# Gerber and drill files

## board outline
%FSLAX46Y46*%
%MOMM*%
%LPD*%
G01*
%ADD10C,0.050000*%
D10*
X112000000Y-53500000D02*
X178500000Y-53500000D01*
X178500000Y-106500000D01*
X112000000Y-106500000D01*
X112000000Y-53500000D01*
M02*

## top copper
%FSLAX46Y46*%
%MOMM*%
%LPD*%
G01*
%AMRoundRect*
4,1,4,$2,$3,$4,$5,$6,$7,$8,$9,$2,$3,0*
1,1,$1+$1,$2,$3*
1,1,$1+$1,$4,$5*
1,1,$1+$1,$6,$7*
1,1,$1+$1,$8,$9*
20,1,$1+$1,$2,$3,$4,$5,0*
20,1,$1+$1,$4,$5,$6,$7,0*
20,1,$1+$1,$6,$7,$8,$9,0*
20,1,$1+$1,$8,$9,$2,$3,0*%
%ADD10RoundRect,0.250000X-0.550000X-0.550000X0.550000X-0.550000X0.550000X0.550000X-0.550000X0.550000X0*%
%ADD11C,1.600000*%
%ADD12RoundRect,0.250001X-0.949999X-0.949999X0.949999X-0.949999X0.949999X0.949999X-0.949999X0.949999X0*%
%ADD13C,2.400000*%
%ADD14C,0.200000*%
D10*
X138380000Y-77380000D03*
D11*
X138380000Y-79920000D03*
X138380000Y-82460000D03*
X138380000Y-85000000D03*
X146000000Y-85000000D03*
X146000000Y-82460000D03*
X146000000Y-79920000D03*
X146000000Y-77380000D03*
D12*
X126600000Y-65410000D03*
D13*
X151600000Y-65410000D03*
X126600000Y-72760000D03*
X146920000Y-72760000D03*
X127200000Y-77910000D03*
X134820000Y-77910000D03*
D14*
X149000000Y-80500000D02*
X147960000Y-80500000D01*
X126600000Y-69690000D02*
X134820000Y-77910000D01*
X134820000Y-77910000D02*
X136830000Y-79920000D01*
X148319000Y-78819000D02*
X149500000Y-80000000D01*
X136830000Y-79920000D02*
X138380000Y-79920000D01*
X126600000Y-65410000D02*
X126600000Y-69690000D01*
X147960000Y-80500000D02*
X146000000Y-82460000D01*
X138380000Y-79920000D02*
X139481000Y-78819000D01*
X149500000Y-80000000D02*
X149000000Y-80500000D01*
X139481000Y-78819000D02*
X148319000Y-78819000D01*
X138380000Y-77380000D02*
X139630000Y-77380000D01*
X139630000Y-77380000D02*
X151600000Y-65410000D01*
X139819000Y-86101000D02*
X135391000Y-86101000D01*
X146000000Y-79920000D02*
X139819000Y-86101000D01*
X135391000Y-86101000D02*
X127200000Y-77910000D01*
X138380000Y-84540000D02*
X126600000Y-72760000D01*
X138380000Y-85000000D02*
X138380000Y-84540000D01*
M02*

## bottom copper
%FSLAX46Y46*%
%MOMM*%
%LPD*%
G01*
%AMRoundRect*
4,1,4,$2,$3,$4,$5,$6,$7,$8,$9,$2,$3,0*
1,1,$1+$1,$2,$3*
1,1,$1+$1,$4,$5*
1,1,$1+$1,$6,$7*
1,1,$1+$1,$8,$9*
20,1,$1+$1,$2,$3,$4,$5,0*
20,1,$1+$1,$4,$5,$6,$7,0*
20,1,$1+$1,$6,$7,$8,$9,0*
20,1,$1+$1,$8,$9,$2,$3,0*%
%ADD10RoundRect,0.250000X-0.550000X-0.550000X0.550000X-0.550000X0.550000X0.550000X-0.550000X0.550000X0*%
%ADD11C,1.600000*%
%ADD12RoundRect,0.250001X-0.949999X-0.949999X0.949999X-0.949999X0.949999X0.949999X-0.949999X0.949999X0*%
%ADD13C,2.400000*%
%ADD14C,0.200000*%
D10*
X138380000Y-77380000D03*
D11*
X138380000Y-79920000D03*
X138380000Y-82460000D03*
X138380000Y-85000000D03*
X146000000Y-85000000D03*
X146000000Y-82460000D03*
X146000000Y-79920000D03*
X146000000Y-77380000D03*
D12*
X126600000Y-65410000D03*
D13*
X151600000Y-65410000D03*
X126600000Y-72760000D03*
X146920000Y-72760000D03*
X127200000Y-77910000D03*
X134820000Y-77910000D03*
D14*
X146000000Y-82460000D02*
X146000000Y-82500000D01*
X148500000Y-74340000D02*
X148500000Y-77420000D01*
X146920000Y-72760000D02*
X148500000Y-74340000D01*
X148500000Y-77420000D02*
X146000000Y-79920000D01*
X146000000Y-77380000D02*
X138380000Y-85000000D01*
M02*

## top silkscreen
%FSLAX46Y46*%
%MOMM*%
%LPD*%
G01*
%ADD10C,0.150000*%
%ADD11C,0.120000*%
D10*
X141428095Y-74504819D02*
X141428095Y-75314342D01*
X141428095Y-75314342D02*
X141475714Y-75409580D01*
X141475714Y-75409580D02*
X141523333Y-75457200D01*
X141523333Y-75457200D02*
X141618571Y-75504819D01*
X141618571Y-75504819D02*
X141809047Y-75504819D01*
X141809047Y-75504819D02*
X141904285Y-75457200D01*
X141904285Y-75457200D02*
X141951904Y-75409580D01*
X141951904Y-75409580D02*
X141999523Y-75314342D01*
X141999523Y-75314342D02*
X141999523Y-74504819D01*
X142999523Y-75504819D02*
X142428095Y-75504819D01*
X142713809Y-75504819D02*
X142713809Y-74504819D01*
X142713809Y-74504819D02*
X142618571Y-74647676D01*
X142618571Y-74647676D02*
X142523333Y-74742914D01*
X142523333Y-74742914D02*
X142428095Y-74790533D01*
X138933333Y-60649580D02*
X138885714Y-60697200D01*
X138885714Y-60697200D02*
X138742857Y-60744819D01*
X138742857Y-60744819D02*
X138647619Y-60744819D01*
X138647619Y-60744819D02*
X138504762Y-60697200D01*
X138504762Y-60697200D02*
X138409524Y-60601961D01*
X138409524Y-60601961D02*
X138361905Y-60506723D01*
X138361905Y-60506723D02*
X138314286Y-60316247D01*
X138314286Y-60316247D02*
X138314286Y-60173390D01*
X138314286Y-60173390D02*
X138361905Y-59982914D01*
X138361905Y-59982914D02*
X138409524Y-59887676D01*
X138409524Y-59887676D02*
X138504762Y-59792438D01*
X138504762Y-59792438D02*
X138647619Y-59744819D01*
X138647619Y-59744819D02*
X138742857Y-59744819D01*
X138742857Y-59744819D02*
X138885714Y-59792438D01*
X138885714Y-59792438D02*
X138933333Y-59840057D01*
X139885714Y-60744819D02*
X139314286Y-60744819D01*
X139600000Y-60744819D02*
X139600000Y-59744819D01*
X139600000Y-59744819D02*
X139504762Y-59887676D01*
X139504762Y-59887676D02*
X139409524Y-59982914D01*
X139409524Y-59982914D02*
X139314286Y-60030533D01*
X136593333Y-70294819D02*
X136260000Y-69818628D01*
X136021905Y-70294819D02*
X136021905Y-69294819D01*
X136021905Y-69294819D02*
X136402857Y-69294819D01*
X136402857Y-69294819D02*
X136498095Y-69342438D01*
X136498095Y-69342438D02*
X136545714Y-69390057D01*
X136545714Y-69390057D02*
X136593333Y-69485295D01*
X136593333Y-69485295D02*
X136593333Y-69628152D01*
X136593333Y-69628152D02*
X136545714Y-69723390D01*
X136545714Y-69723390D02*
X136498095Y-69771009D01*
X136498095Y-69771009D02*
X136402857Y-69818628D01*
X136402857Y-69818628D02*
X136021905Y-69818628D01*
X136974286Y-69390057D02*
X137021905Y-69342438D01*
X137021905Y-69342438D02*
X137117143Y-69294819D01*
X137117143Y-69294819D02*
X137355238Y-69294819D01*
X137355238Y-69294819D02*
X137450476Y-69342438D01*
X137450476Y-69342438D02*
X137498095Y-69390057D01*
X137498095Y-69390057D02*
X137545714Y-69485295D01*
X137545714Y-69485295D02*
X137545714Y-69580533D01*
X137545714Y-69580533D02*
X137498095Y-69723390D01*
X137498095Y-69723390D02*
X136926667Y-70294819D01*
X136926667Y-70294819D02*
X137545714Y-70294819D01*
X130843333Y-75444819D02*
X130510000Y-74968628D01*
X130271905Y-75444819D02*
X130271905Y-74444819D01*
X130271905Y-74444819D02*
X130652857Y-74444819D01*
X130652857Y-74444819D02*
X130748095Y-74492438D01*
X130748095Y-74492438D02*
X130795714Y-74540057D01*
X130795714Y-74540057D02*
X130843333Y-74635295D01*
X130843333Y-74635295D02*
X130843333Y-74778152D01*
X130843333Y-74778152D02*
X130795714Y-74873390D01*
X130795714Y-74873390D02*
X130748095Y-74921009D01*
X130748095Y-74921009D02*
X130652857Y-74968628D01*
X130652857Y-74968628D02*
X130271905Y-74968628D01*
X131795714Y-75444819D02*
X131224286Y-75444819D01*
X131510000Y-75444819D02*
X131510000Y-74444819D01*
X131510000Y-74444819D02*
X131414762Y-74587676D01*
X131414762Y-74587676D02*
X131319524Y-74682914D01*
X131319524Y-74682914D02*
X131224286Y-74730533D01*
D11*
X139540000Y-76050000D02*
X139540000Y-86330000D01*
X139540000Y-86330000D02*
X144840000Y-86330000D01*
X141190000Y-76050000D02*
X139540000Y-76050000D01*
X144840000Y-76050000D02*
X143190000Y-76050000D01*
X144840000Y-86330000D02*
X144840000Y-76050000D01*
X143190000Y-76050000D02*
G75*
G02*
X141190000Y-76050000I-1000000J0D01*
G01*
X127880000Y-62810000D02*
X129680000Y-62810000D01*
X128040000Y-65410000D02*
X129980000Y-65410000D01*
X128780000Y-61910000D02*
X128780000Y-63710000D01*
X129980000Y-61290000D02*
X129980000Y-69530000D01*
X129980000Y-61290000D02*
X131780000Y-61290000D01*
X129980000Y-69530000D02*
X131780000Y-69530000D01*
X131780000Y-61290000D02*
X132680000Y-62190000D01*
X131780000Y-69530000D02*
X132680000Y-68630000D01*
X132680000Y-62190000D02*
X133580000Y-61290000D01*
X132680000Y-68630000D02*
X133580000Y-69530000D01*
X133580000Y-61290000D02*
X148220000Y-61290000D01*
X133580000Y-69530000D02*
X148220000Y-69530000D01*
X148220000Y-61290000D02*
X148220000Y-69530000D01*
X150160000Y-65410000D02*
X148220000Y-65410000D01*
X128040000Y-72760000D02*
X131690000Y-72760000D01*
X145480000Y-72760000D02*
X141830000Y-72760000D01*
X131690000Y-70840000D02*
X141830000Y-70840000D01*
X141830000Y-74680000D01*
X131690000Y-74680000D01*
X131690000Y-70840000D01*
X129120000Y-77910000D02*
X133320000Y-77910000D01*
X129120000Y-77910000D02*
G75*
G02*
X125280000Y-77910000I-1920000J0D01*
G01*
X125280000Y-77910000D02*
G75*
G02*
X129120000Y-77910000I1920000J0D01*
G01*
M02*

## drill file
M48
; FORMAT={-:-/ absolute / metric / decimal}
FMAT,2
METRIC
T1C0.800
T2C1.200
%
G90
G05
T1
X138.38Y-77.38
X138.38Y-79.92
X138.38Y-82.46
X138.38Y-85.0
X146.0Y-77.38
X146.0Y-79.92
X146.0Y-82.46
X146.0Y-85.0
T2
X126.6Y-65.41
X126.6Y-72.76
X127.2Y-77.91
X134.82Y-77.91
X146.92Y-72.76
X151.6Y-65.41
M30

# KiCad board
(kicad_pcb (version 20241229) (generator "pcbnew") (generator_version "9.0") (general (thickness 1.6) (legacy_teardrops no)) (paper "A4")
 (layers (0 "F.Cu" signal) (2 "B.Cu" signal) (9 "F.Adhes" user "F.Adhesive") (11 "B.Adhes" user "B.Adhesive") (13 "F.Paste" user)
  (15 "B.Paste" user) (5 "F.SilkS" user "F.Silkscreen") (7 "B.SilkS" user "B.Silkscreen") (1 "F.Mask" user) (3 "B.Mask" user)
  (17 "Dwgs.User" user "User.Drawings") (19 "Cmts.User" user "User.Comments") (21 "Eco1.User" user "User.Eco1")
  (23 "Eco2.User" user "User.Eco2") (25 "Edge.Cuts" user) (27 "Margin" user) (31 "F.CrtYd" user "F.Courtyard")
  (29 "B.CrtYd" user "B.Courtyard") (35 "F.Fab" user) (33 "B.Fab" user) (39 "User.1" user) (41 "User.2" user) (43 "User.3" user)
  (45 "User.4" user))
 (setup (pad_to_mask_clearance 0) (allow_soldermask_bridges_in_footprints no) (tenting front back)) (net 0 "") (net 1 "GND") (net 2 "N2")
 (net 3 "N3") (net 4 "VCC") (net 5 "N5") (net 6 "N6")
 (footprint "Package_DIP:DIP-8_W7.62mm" (layer "F.Cu") (at 138.38 77.38)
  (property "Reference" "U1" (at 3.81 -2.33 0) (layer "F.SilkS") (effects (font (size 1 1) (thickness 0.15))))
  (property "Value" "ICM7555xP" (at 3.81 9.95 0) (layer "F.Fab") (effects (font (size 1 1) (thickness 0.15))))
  (fp_line (start 1.16 -1.33) (end 1.16 8.95) (stroke (width 0.12) (type solid)) (layer "F.SilkS"))
  (fp_line (start 1.16 8.95) (end 6.46 8.95) (stroke (width 0.12) (type solid)) (layer "F.SilkS"))
  (fp_line (start 2.81 -1.33) (end 1.16 -1.33) (stroke (width 0.12) (type solid)) (layer "F.SilkS"))
  (fp_line (start 6.46 -1.33) (end 4.81 -1.33) (stroke (width 0.12) (type solid)) (layer "F.SilkS"))
  (fp_line (start 6.46 8.95) (end 6.46 -1.33) (stroke (width 0.12) (type solid)) (layer "F.SilkS"))
  (fp_arc (start 4.81 -1.33) (mid 3.81 -0.33) (end 2.81 -1.33) (stroke (width 0.12) (type solid)) (layer "F.SilkS"))
  (pad "1" thru_hole roundrect (at 0 0) (size 1.6 1.6) (drill 0.8) (layers "*.Cu" "*.Mask") (remove_unused_layers no)
   (roundrect_rratio 0.15625) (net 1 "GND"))
  (pad "2" thru_hole circle (at 0 2.54) (size 1.6 1.6) (drill 0.8) (layers "*.Cu" "*.Mask") (remove_unused_layers no) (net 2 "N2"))
  (pad "3" thru_hole circle (at 0 5.08) (size 1.6 1.6) (drill 0.8) (layers "*.Cu" "*.Mask") (remove_unused_layers no) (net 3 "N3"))
  (pad "4" thru_hole circle (at 0 7.62) (size 1.6 1.6) (drill 0.8) (layers "*.Cu" "*.Mask") (remove_unused_layers no) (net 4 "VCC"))
  (pad "5" thru_hole circle (at 7.62 7.62) (size 1.6 1.6) (drill 0.8) (layers "*.Cu" "*.Mask") (remove_unused_layers no) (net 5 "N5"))
  (pad "6" thru_hole circle (at 7.62 5.08) (size 1.6 1.6) (drill 0.8) (layers "*.Cu" "*.Mask") (remove_unused_layers no) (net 2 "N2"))
  (pad "7" thru_hole circle (at 7.62 2.54) (size 1.6 1.6) (drill 0.8) (layers "*.Cu" "*.Mask") (remove_unused_layers no) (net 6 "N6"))
  (pad "8" thru_hole circle (at 7.62 0) (size 1.6 1.6) (drill 0.8) (layers "*.Cu" "*.Mask") (remove_unused_layers no) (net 4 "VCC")))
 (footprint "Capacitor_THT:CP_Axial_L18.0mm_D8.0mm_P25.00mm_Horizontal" (layer "F.Cu") (at 126.6 65.41)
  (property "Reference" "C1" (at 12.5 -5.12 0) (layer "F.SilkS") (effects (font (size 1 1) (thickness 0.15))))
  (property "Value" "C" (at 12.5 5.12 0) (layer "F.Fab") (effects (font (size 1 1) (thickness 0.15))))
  (fp_line (start 1.28 -2.6) (end 3.08 -2.6) (stroke (width 0.12) (type solid)) (layer "F.SilkS"))
  (fp_line (start 1.44 0) (end 3.38 0) (stroke (width 0.12) (type solid)) (layer "F.SilkS"))
  (fp_line (start 2.18 -3.5) (end 2.18 -1.7) (stroke (width 0.12) (type solid)) (layer "F.SilkS"))
  (fp_line (start 3.38 -4.12) (end 3.38 4.12) (stroke (width 0.12) (type solid)) (layer "F.SilkS"))
  (fp_line (start 3.38 -4.12) (end 5.18 -4.12) (stroke (width 0.12) (type solid)) (layer "F.SilkS"))
  (fp_line (start 3.38 4.12) (end 5.18 4.12) (stroke (width 0.12) (type solid)) (layer "F.SilkS"))
  (fp_line (start 5.18 -4.12) (end 6.08 -3.22) (stroke (width 0.12) (type solid)) (layer "F.SilkS"))
  (fp_line (start 5.18 4.12) (end 6.08 3.22) (stroke (width 0.12) (type solid)) (layer "F.SilkS"))
  (fp_line (start 6.08 -3.22) (end 6.98 -4.12) (stroke (width 0.12) (type solid)) (layer "F.SilkS"))
  (fp_line (start 6.08 3.22) (end 6.98 4.12) (stroke (width 0.12) (type solid)) (layer "F.SilkS"))
  (fp_line (start 6.98 -4.12) (end 21.62 -4.12) (stroke (width 0.12) (type solid)) (layer "F.SilkS"))
  (fp_line (start 6.98 4.12) (end 21.62 4.12) (stroke (width 0.12) (type solid)) (layer "F.SilkS"))
  (fp_line (start 21.62 -4.12) (end 21.62 4.12) (stroke (width 0.12) (type solid)) (layer "F.SilkS"))
  (fp_line (start 23.56 0) (end 21.62 0) (stroke (width 0.12) (type solid)) (layer "F.SilkS"))
  (pad "1" thru_hole roundrect (at 0 0) (size 2.4 2.4) (drill 1.2) (layers "*.Cu" "*.Mask") (remove_unused_layers no)
   (roundrect_rratio 0.104167) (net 2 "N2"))
  (pad "2" thru_hole circle (at 25 0) (size 2.4 2.4) (drill 1.2) (layers "*.Cu" "*.Mask") (remove_unused_layers no) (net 1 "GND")))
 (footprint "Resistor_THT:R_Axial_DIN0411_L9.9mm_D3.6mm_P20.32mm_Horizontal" (layer "F.Cu") (at 126.6 72.76)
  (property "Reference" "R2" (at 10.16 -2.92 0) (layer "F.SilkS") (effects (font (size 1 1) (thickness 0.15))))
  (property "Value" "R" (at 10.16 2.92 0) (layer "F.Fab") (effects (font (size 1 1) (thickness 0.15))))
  (fp_line (start 1.44 0) (end 5.09 0) (stroke (width 0.12) (type solid)) (layer "F.SilkS"))
  (fp_line (start 18.88 0) (end 15.23 0) (stroke (width 0.12) (type solid)) (layer "F.SilkS"))
  (fp_rect (start 5.09 -1.92) (end 15.23 1.92) (stroke (width 0.12) (type solid)) (fill no) (layer "F.SilkS"))
  (pad "1" thru_hole circle (at 0 0) (size 2.4 2.4) (drill 1.2) (layers "*.Cu" "*.Mask") (remove_unused_layers no) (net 4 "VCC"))
  (pad "2" thru_hole circle (at 20.32 0) (size 2.4 2.4) (drill 1.2) (layers "*.Cu" "*.Mask") (remove_unused_layers no) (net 6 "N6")))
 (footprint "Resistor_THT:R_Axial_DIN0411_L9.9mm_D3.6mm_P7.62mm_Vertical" (layer "F.Cu") (at 127.2 77.91)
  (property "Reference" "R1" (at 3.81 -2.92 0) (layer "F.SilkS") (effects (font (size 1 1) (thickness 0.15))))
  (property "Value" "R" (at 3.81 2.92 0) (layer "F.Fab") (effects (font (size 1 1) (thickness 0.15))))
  (fp_line (start 1.92 0) (end 6.12 0) (stroke (width 0.12) (type solid)) (layer "F.SilkS"))
  (fp_circle (center 0 0) (end 1.92 0) (stroke (width 0.12) (type solid)) (fill no) (layer "F.SilkS"))
  (pad "1" thru_hole circle (at 0 0) (size 2.4 2.4) (drill 1.2) (layers "*.Cu" "*.Mask") (remove_unused_layers no) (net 6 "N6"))
  (pad "2" thru_hole circle (at 7.62 0) (size 2.4 2.4) (drill 1.2) (layers "*.Cu" "*.Mask") (remove_unused_layers no) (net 2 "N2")))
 (gr_rect (start 112 53.5) (end 178.5 106.5) (stroke (width 0.05) (type default)) (fill no) (layer "Edge.Cuts"))
 (segment (start 149 80.5) (end 147.96 80.5) (width 0.2) (layer "F.Cu") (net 2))
 (segment (start 126.6 69.69) (end 134.82 77.91) (width 0.2) (layer "F.Cu") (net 2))
 (segment (start 134.82 77.91) (end 136.83 79.92) (width 0.2) (layer "F.Cu") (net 2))
 (segment (start 148.319 78.819) (end 149.5 80) (width 0.2) (layer "F.Cu") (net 2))
 (segment (start 136.83 79.92) (end 138.38 79.92) (width 0.2) (layer "F.Cu") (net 2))
 (segment (start 126.6 65.41) (end 126.6 69.69) (width 0.2) (layer "F.Cu") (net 2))
 (segment (start 147.96 80.5) (end 146 82.46) (width 0.2) (layer "F.Cu") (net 2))
 (segment (start 138.38 79.92) (end 139.481 78.819) (width 0.2) (layer "F.Cu") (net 2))
 (segment (start 149.5 80) (end 149 80.5) (width 0.2) (layer "F.Cu") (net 2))
 (segment (start 139.481 78.819) (end 148.319 78.819) (width 0.2) (layer "F.Cu") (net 2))
 (segment (start 146 82.46) (end 146 82.5) (width 0.2) (layer "B.Cu") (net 2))
 (segment (start 138.38 77.38) (end 139.63 77.38) (width 0.2) (layer "F.Cu") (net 1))
 (segment (start 139.63 77.38) (end 151.6 65.41) (width 0.2) (layer "F.Cu") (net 1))
 (segment (start 139.819 86.101) (end 135.391 86.101) (width 0.2) (layer "F.Cu") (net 6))
 (segment (start 146 79.92) (end 139.819 86.101) (width 0.2) (layer "F.Cu") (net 6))
 (segment (start 135.391 86.101) (end 127.2 77.91) (width 0.2) (layer "F.Cu") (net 6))
 (segment (start 148.5 74.34) (end 148.5 77.42) (width 0.2) (layer "B.Cu") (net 6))
 (segment (start 146.92 72.76) (end 148.5 74.34) (width 0.2) (layer "B.Cu") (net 6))
 (segment (start 148.5 77.42) (end 146 79.92) (width 0.2) (layer "B.Cu") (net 6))
 (segment (start 138.38 84.54) (end 126.6 72.76) (width 0.2) (layer "F.Cu") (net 4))
 (segment (start 138.38 85) (end 138.38 84.54) (width 0.2) (layer "F.Cu") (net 4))
 (segment (start 146 77.38) (end 138.38 85) (width 0.2) (layer "B.Cu") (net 4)))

